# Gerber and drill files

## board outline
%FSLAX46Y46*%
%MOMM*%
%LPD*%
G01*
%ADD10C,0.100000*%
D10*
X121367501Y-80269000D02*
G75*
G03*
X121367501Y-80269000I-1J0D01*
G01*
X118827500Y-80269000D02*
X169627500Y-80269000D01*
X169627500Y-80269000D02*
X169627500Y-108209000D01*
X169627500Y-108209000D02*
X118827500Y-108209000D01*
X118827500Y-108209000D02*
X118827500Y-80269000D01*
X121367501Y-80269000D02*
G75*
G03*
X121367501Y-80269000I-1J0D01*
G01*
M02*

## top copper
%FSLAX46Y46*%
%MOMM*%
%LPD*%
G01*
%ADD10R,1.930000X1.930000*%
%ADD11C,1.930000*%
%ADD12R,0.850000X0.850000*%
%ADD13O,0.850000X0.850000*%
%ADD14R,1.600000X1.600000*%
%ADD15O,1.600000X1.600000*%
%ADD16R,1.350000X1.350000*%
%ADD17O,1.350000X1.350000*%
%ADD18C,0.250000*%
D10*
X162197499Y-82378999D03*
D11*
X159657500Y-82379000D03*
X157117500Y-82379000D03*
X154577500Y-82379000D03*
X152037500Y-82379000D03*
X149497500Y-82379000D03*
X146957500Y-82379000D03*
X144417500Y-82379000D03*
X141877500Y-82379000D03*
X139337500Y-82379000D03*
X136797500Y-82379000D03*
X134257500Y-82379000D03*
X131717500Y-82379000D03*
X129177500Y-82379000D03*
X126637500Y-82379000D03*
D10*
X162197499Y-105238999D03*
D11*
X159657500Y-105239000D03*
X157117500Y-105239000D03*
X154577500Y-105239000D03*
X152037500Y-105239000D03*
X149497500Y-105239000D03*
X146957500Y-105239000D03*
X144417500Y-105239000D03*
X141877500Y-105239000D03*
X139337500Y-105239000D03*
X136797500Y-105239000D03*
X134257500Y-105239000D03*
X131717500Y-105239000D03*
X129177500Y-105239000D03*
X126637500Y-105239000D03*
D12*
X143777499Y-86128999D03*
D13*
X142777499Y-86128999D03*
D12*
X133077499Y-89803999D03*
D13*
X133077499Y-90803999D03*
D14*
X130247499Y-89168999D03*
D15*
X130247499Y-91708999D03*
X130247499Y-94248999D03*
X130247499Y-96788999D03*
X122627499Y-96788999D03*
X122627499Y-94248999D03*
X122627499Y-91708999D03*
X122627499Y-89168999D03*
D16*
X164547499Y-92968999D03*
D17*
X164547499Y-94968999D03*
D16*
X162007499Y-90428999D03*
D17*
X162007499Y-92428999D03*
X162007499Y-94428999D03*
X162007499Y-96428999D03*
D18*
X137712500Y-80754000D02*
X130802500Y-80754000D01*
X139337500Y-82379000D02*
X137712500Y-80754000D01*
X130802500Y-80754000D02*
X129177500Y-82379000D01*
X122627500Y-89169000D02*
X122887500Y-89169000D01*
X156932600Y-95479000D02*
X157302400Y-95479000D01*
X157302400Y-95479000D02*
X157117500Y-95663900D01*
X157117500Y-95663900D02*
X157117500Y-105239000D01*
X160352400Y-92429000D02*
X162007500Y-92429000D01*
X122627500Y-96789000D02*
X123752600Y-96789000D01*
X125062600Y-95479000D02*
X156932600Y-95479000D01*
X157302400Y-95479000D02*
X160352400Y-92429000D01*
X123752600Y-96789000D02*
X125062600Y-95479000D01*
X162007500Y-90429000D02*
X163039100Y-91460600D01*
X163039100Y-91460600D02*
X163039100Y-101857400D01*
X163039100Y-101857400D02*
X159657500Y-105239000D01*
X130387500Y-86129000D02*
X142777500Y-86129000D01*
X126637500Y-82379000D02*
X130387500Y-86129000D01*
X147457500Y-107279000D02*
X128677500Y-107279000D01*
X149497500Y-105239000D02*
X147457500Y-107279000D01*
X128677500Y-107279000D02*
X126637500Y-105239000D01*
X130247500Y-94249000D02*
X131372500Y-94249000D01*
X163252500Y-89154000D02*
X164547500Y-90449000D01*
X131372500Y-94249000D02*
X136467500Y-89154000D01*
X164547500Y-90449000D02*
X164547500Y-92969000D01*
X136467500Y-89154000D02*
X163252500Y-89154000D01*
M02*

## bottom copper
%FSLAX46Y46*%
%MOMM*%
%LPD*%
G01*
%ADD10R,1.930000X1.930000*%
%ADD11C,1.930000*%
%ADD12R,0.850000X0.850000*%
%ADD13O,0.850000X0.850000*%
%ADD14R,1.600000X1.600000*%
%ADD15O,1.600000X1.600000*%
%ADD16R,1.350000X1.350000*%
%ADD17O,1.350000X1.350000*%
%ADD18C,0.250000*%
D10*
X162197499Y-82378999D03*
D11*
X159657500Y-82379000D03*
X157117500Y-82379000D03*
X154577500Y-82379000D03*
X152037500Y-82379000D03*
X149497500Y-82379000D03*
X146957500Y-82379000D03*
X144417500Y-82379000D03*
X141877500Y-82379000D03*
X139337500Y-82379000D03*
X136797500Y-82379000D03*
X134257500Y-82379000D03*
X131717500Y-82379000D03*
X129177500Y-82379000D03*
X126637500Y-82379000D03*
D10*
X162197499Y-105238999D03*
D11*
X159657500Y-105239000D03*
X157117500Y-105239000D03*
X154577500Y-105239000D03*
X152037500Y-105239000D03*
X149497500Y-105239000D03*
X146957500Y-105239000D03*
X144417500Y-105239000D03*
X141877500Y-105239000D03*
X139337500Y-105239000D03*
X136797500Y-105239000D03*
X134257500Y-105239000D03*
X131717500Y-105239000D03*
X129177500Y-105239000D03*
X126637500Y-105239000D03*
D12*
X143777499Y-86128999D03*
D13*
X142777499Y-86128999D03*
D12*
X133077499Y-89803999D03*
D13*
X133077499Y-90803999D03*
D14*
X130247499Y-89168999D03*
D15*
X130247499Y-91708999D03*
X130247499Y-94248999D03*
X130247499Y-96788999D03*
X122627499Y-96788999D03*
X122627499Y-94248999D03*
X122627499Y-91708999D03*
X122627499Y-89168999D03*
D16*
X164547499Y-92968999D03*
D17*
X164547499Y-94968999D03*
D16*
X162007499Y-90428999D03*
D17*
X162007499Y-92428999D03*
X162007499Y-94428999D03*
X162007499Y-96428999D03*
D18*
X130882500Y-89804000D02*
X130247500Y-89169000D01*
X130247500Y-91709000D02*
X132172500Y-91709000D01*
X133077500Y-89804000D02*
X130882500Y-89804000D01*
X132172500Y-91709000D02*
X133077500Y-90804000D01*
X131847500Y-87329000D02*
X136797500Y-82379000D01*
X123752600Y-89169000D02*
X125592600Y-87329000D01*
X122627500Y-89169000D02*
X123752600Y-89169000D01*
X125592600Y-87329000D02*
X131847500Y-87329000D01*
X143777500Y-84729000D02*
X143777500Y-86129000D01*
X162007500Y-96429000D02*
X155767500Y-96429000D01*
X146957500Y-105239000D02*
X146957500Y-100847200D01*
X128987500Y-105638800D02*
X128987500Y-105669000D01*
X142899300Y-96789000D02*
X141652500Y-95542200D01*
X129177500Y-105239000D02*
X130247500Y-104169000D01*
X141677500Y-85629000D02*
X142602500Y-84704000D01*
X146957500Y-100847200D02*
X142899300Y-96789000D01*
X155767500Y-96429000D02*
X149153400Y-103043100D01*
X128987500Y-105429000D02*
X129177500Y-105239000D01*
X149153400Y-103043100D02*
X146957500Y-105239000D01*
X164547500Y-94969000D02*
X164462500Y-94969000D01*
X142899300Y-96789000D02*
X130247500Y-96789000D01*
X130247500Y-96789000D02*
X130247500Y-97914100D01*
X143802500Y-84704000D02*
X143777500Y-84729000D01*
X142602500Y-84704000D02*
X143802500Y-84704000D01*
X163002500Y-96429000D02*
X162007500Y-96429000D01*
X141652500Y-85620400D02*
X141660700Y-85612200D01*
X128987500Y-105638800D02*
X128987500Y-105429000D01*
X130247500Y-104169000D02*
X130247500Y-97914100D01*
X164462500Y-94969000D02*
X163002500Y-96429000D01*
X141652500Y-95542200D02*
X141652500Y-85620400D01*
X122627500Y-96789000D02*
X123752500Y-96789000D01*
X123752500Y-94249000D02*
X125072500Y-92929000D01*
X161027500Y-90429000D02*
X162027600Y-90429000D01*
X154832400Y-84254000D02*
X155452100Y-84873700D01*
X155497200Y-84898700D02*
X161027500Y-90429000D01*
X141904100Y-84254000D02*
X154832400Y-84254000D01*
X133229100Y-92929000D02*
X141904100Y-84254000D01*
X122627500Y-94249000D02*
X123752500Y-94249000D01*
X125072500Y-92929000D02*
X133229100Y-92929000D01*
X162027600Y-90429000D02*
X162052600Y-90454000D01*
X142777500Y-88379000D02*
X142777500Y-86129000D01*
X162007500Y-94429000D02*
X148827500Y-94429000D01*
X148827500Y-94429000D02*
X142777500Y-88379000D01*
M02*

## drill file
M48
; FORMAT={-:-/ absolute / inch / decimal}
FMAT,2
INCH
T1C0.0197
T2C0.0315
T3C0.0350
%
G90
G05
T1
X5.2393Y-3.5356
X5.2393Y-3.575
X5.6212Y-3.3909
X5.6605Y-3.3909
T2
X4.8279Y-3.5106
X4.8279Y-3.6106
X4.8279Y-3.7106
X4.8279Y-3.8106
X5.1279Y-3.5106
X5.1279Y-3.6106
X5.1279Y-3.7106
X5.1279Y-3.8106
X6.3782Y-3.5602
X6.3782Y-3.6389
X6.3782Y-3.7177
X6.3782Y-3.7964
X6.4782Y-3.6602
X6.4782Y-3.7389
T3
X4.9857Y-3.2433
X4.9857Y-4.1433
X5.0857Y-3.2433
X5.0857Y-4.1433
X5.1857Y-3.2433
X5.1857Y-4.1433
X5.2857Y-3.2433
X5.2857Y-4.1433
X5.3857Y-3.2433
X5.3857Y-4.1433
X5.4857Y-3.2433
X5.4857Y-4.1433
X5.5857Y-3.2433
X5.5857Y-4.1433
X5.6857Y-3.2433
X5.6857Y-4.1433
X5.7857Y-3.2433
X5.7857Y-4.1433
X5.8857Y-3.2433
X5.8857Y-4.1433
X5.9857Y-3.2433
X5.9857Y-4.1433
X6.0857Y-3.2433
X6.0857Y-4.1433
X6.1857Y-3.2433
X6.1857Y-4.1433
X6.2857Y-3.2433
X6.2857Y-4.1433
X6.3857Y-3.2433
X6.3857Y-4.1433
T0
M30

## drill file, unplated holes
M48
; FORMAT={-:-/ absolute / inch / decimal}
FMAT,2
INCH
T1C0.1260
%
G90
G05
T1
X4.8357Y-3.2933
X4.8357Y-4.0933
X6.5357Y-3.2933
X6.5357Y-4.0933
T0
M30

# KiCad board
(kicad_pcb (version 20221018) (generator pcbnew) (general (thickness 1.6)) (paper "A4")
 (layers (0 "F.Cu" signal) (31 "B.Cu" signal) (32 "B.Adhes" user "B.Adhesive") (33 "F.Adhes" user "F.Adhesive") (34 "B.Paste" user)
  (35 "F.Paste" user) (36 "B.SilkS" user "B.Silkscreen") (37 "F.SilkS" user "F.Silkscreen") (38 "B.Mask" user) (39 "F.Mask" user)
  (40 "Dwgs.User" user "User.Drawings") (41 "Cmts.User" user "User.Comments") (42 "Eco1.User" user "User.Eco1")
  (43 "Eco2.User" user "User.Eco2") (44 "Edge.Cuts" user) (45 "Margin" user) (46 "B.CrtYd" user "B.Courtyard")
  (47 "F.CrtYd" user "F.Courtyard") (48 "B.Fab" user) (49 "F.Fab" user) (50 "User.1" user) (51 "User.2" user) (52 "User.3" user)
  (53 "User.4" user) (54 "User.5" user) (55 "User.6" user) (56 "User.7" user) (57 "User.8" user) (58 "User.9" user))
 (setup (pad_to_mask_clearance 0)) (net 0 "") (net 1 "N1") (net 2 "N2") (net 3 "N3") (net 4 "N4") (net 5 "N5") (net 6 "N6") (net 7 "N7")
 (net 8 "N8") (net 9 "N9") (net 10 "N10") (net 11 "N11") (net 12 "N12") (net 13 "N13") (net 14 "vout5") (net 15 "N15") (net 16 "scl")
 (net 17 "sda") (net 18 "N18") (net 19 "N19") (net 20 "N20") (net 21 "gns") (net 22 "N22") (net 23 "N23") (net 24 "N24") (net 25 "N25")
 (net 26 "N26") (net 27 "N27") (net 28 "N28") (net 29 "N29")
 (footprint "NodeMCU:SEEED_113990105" (layer "F.Cu") (at 144.4175 93.809 -90)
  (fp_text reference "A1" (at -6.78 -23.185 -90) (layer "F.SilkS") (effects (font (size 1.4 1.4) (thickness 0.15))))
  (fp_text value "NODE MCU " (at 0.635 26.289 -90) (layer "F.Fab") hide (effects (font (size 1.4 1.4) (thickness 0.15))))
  (pad "" np_thru_hole circle (at -10.16 -21.59 270) (size 3.2 3.2) (drill 3.2) (layers "*.Cu" "*.Mask"))
  (pad "" np_thru_hole circle (at -10.16 21.59 270) (size 3.2 3.2) (drill 3.2) (layers "*.Cu" "*.Mask"))
  (pad "" np_thru_hole circle (at 10.16 -21.59 270) (size 3.2 3.2) (drill 3.2) (layers "*.Cu" "*.Mask"))
  (pad "" np_thru_hole circle (at 10.16 21.59 270) (size 3.2 3.2) (drill 3.2) (layers "*.Cu" "*.Mask"))
  (pad "J1_1" thru_hole rect (at -11.43 -17.78 270) (size 1.93 1.93) (drill 0.889) (layers "*.Cu" "*.Mask") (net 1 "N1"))
  (pad "J1_2" thru_hole circle (at -11.43 -15.24 270) (size 1.93 1.93) (drill 0.889) (layers "*.Cu" "*.Mask") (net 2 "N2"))
  (pad "J1_3" thru_hole circle (at -11.43 -12.7 270) (size 1.93 1.93) (drill 0.889) (layers "*.Cu" "*.Mask") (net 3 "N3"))
  (pad "J1_4" thru_hole circle (at -11.43 -10.16 270) (size 1.93 1.93) (drill 0.889) (layers "*.Cu" "*.Mask") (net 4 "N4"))
  (pad "J1_5" thru_hole circle (at -11.43 -7.62 270) (size 1.93 1.93) (drill 0.889) (layers "*.Cu" "*.Mask") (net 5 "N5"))
  (pad "J1_6" thru_hole circle (at -11.43 -5.08 270) (size 1.93 1.93) (drill 0.889) (layers "*.Cu" "*.Mask") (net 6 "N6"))
  (pad "J1_7" thru_hole circle (at -11.43 -2.54 270) (size 1.93 1.93) (drill 0.889) (layers "*.Cu" "*.Mask") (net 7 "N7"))
  (pad "J1_8" thru_hole circle (at -11.43 0 270) (size 1.93 1.93) (drill 0.889) (layers "*.Cu" "*.Mask") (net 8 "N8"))
  (pad "J1_9" thru_hole circle (at -11.43 2.54 270) (size 1.93 1.93) (drill 0.889) (layers "*.Cu" "*.Mask") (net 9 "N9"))
  (pad "J1_10" thru_hole circle (at -11.43 5.08 270) (size 1.93 1.93) (drill 0.889) (layers "*.Cu" "*.Mask") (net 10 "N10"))
  (pad "J1_11" thru_hole circle (at -11.43 7.62 270) (size 1.93 1.93) (drill 0.889) (layers "*.Cu" "*.Mask") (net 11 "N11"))
  (pad "J1_12" thru_hole circle (at -11.43 10.16 270) (size 1.93 1.93) (drill 0.889) (layers "*.Cu" "*.Mask") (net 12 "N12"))
  (pad "J1_13" thru_hole circle (at -11.43 12.7 270) (size 1.93 1.93) (drill 0.889) (layers "*.Cu" "*.Mask") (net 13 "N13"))
  (pad "J1_14" thru_hole circle (at -11.43 15.24 270) (size 1.93 1.93) (drill 0.889) (layers "*.Cu" "*.Mask") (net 10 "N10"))
  (pad "J1_15" thru_hole circle (at -11.43 17.78 270) (size 1.93 1.93) (drill 0.889) (layers "*.Cu" "*.Mask") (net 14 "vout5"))
  (pad "J2_1" thru_hole rect (at 11.43 -17.78 270) (size 1.93 1.93) (drill 0.889) (layers "*.Cu" "*.Mask") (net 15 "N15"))
  (pad "J2_2" thru_hole circle (at 11.43 -15.24 270) (size 1.93 1.93) (drill 0.889) (layers "*.Cu" "*.Mask") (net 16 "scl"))
  (pad "J2_3" thru_hole circle (at 11.43 -12.7 270) (size 1.93 1.93) (drill 0.889) (layers "*.Cu" "*.Mask") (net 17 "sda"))
  (pad "J2_4" thru_hole circle (at 11.43 -10.16 270) (size 1.93 1.93) (drill 0.889) (layers "*.Cu" "*.Mask") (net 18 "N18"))
  (pad "J2_5" thru_hole circle (at 11.43 -7.62 270) (size 1.93 1.93) (drill 0.889) (layers "*.Cu" "*.Mask") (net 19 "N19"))
  (pad "J2_6" thru_hole circle (at 11.43 -5.08 270) (size 1.93 1.93) (drill 0.889) (layers "*.Cu" "*.Mask") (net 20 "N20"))
  (pad "J2_7" thru_hole circle (at 11.43 -2.54 270) (size 1.93 1.93) (drill 0.889) (layers "*.Cu" "*.Mask") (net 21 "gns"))
  (pad "J2_8" thru_hole circle (at 11.43 0 270) (size 1.93 1.93) (drill 0.889) (layers "*.Cu" "*.Mask") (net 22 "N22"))
  (pad "J2_9" thru_hole circle (at 11.43 2.54 270) (size 1.93 1.93) (drill 0.889) (layers "*.Cu" "*.Mask") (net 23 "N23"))
  (pad "J2_10" thru_hole circle (at 11.43 5.08 270) (size 1.93 1.93) (drill 0.889) (layers "*.Cu" "*.Mask") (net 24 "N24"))
  (pad "J2_11" thru_hole circle (at 11.43 7.62 270) (size 1.93 1.93) (drill 0.889) (layers "*.Cu" "*.Mask") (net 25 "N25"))
  (pad "J2_12" thru_hole circle (at 11.43 10.16 270) (size 1.93 1.93) (drill 0.889) (layers "*.Cu" "*.Mask") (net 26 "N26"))
  (pad "J2_13" thru_hole circle (at 11.43 12.7 270) (size 1.93 1.93) (drill 0.889) (layers "*.Cu" "*.Mask") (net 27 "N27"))
  (pad "J2_14" thru_hole circle (at 11.43 15.24 270) (size 1.93 1.93) (drill 0.889) (layers "*.Cu" "*.Mask") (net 21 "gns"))
  (pad "J2_15" thru_hole circle (at 11.43 17.78 270) (size 1.93 1.93) (drill 0.889) (layers "*.Cu" "*.Mask") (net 20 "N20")))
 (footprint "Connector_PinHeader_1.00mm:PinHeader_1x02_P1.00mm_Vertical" (layer "F.Cu") (at 143.7775 86.129 -90)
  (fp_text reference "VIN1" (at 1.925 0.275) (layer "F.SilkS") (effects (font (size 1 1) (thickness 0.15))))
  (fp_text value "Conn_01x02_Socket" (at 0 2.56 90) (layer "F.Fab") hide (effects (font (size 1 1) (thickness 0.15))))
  (pad "1" thru_hole rect (at 0 0 270) (size 0.85 0.85) (drill 0.5) (layers "*.Cu" "*.Mask") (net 21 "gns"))
  (pad "2" thru_hole oval (at 0 1 270) (size 0.85 0.85) (drill 0.5) (layers "*.Cu" "*.Mask") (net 14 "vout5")))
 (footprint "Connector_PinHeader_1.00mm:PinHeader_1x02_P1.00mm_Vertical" (layer "F.Cu") (at 133.0775 89.804)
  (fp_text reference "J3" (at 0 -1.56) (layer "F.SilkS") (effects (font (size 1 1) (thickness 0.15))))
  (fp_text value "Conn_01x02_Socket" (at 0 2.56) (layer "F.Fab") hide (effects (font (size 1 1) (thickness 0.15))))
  (pad "1" thru_hole rect (at 0 0) (size 0.85 0.85) (drill 0.5) (layers "*.Cu" "*.Mask"))
  (pad "2" thru_hole oval (at 0 1) (size 0.85 0.85) (drill 0.5) (layers "*.Cu" "*.Mask")))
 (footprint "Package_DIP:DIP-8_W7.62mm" (layer "B.Cu") (at 130.2475 89.169 180)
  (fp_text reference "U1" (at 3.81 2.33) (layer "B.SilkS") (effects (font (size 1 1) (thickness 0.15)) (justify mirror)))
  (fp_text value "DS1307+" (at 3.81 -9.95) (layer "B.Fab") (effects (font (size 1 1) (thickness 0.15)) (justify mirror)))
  (pad "1" thru_hole rect (at 0 0 180) (size 1.6 1.6) (drill 0.8) (layers "*.Cu" "*.Mask"))
  (pad "2" thru_hole oval (at 0 -2.54 180) (size 1.6 1.6) (drill 0.8) (layers "*.Cu" "*.Mask"))
  (pad "3" thru_hole oval (at 0 -5.08 180) (size 1.6 1.6) (drill 0.8) (layers "*.Cu" "*.Mask") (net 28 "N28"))
  (pad "4" thru_hole oval (at 0 -7.62 180) (size 1.6 1.6) (drill 0.8) (layers "*.Cu" "*.Mask") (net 21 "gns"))
  (pad "5" thru_hole oval (at 7.62 -7.62 180) (size 1.6 1.6) (drill 0.8) (layers "*.Cu" "*.Mask") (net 17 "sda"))
  (pad "6" thru_hole oval (at 7.62 -5.08 180) (size 1.6 1.6) (drill 0.8) (layers "*.Cu" "*.Mask") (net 16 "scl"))
  (pad "7" thru_hole oval (at 7.62 -2.54 180) (size 1.6 1.6) (drill 0.8) (layers "*.Cu" "*.Mask") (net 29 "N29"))
  (pad "8" thru_hole oval (at 7.62 0 180) (size 1.6 1.6) (drill 0.8) (layers "*.Cu" "*.Mask") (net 11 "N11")))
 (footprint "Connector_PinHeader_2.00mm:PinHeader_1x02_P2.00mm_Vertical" (layer "B.Cu") (at 164.5475 92.969 180)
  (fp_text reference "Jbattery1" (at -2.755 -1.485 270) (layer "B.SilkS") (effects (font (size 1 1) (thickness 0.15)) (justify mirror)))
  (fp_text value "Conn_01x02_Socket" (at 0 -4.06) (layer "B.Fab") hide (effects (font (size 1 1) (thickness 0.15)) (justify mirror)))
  (pad "1" thru_hole rect (at 0 0 180) (size 1.35 1.35) (drill 0.8) (layers "*.Cu" "*.Mask") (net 28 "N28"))
  (pad "2" thru_hole oval (at 0 -2 180) (size 1.35 1.35) (drill 0.8) (layers "*.Cu" "*.Mask") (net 21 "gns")))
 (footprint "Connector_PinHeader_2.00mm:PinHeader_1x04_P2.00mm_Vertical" (layer "B.Cu") (at 162.0075 90.429 180)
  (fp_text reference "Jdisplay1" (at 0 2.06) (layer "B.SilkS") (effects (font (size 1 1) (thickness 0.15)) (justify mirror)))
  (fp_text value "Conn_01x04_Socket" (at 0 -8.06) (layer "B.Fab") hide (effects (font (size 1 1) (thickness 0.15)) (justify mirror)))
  (pad "1" thru_hole rect (at 0 0 180) (size 1.35 1.35) (drill 0.8) (layers "*.Cu" "*.Mask") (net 16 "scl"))
  (pad "2" thru_hole oval (at 0 -2 180) (size 1.35 1.35) (drill 0.8) (layers "*.Cu" "*.Mask") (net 17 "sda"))
  (pad "3" thru_hole oval (at 0 -4 180) (size 1.35 1.35) (drill 0.8) (layers "*.Cu" "*.Mask") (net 14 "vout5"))
  (pad "4" thru_hole oval (at 0 -6 180) (size 1.35 1.35) (drill 0.8) (layers "*.Cu" "*.Mask") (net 21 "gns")))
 (gr_circle (center 121.3675 80.269) (end 121.3675 80.269) (stroke (width 0.1) (type default)) (fill none) (layer "Edge.Cuts"))
 (gr_rect (start 118.8275 80.269) (end 169.6275 108.209) (stroke (width 0.1) (type default)) (fill none) (layer "Edge.Cuts"))
 (gr_circle (center 121.3675 80.269) (end 121.3675 80.269) (stroke (width 0.1) (type default)) (fill none) (layer "Edge.Cuts"))
 (segment (start 130.8825 89.804) (end 130.2475 89.169) (width 0.25) (layer "B.Cu") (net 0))
 (segment (start 130.2475 91.709) (end 132.1725 91.709) (width 0.25) (layer "B.Cu") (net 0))
 (segment (start 133.0775 89.804) (end 130.8825 89.804) (width 0.25) (layer "B.Cu") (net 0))
 (segment (start 132.1725 91.709) (end 133.0775 90.804) (width 0.25) (layer "B.Cu") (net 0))
 (segment (start 137.7125 80.754) (end 130.8025 80.754) (width 0.25) (layer "F.Cu") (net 10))
 (segment (start 139.3375 82.379) (end 137.7125 80.754) (width 0.25) (layer "F.Cu") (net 10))
 (segment (start 130.8025 80.754) (end 129.1775 82.379) (width 0.25) (layer "F.Cu") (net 10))
 (segment (start 122.6275 89.169) (end 122.8875 89.169) (width 0.25) (layer "F.Cu") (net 11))
 (segment (start 131.8475 87.329) (end 136.7975 82.379) (width 0.25) (layer "B.Cu") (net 11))
 (segment (start 123.7526 89.169) (end 125.5926 87.329) (width 0.25) (layer "B.Cu") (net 11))
 (segment (start 122.6275 89.169) (end 123.7526 89.169) (width 0.25) (layer "B.Cu") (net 11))
 (segment (start 125.5926 87.329) (end 131.8475 87.329) (width 0.25) (layer "B.Cu") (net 11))
 (segment (start 143.7775 84.729) (end 143.7775 86.129) (width 0.25) (layer "B.Cu") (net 21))
 (segment (start 162.0075 96.429) (end 155.7675 96.429) (width 0.25) (layer "B.Cu") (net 21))
 (segment (start 146.9575 105.239) (end 146.9575 100.8472) (width 0.25) (layer "B.Cu") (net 21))
 (segment (start 128.9875 105.6388) (end 128.9875 105.669) (width 0.25) (layer "B.Cu") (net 21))
 (segment (start 142.8993 96.789) (end 141.6525 95.5422) (width 0.25) (layer "B.Cu") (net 21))
 (segment (start 129.1775 105.239) (end 130.2475 104.169) (width 0.25) (layer "B.Cu") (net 21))
 (segment (start 141.6775 85.629) (end 142.6025 84.704) (width 0.25) (layer "B.Cu") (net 21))
 (segment (start 146.9575 100.8472) (end 142.8993 96.789) (width 0.25) (layer "B.Cu") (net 21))
 (segment (start 155.7675 96.429) (end 149.1534 103.0431) (width 0.25) (layer "B.Cu") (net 21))
 (segment (start 128.9875 105.429) (end 129.1775 105.239) (width 0.25) (layer "B.Cu") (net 21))
 (segment (start 149.1534 103.0431) (end 146.9575 105.239) (width 0.25) (layer "B.Cu") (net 21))
 (segment (start 164.5475 94.969) (end 164.4625 94.969) (width 0.25) (layer "B.Cu") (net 21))
 (segment (start 142.8993 96.789) (end 130.2475 96.789) (width 0.25) (layer "B.Cu") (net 21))
 (segment (start 130.2475 96.789) (end 130.2475 97.9141) (width 0.25) (layer "B.Cu") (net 21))
 (segment (start 143.8025 84.704) (end 143.7775 84.729) (width 0.25) (layer "B.Cu") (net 21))
 (segment (start 142.6025 84.704) (end 143.8025 84.704) (width 0.25) (layer "B.Cu") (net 21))
 (segment (start 163.0025 96.429) (end 162.0075 96.429) (width 0.25) (layer "B.Cu") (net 21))
 (segment (start 141.6525 85.6204) (end 141.6607 85.6122) (width 0.25) (layer "B.Cu") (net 21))
 (segment (start 128.9875 105.6388) (end 128.9875 105.429) (width 0.25) (layer "B.Cu") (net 21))
 (segment (start 130.2475 104.169) (end 130.2475 97.9141) (width 0.25) (layer "B.Cu") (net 21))
 (segment (start 164.4625 94.969) (end 163.0025 96.429) (width 0.25) (layer "B.Cu") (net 21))
 (segment (start 141.6525 95.5422) (end 141.6525 85.6204) (width 0.25) (layer "B.Cu") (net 21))
 (segment (start 156.9326 95.479) (end 157.3024 95.479) (width 0.25) (layer "F.Cu") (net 17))
 (segment (start 157.3024 95.479) (end 157.1175 95.6639) (width 0.25) (layer "F.Cu") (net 17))
 (segment (start 157.1175 95.6639) (end 157.1175 105.239) (width 0.25) (layer "F.Cu") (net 17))
 (segment (start 160.3524 92.429) (end 162.0075 92.429) (width 0.25) (layer "F.Cu") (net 17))
 (segment (start 122.6275 96.789) (end 123.7526 96.789) (width 0.25) (layer "F.Cu") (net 17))
 (segment (start 125.0626 95.479) (end 156.9326 95.479) (width 0.25) (layer "F.Cu") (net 17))
 (segment (start 157.3024 95.479) (end 160.3524 92.429) (width 0.25) (layer "F.Cu") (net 17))
 (segment (start 123.7526 96.789) (end 125.0626 95.479) (width 0.25) (layer "F.Cu") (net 17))
 (segment (start 122.6275 96.789) (end 123.7525 96.789) (width 0.25) (layer "B.Cu") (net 17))
 (segment (start 162.0075 90.429) (end 163.0391 91.4606) (width 0.25) (layer "F.Cu") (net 16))
 (segment (start 163.0391 91.4606) (end 163.0391 101.8574) (width 0.25) (layer "F.Cu") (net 16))
 (segment (start 163.0391 101.8574) (end 159.6575 105.239) (width 0.25) (layer "F.Cu") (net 16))
 (segment (start 123.7525 94.249) (end 125.0725 92.929) (width 0.25) (layer "B.Cu") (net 16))
 (segment (start 161.0275 90.429) (end 162.0276 90.429) (width 0.25) (layer "B.Cu") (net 16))
 (segment (start 154.8324 84.254) (end 155.4521 84.8737) (width 0.25) (layer "B.Cu") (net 16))
 (segment (start 155.4972 84.8987) (end 161.0275 90.429) (width 0.25) (layer "B.Cu") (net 16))
 (segment (start 141.9041 84.254) (end 154.8324 84.254) (width 0.25) (layer "B.Cu") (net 16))
 (segment (start 133.2291 92.929) (end 141.9041 84.254) (width 0.25) (layer "B.Cu") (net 16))
 (segment (start 122.6275 94.249) (end 123.7525 94.249) (width 0.25) (layer "B.Cu") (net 16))
 (segment (start 125.0725 92.929) (end 133.2291 92.929) (width 0.25) (layer "B.Cu") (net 16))
 (segment (start 162.0276 90.429) (end 162.0526 90.454) (width 0.25) (layer "B.Cu") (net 16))
 (segment (start 130.3875 86.129) (end 142.7775 86.129) (width 0.25) (layer "F.Cu") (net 14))
 (segment (start 126.6375 82.379) (end 130.3875 86.129) (width 0.25) (layer "F.Cu") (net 14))
 (segment (start 142.7775 88.379) (end 142.7775 86.129) (width 0.25) (layer "B.Cu") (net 14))
 (segment (start 162.0075 94.429) (end 148.8275 94.429) (width 0.25) (layer "B.Cu") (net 14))
 (segment (start 148.8275 94.429) (end 142.7775 88.379) (width 0.25) (layer "B.Cu") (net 14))
 (segment (start 147.4575 107.279) (end 128.6775 107.279) (width 0.25) (layer "F.Cu") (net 20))
 (segment (start 149.4975 105.239) (end 147.4575 107.279) (width 0.25) (layer "F.Cu") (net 20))
 (segment (start 128.6775 107.279) (end 126.6375 105.239) (width 0.25) (layer "F.Cu") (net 20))
 (segment (start 130.2475 94.249) (end 131.3725 94.249) (width 0.25) (layer "F.Cu") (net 28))
 (segment (start 163.2525 89.154) (end 164.5475 90.449) (width 0.25) (layer "F.Cu") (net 28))
 (segment (start 131.3725 94.249) (end 136.4675 89.154) (width 0.25) (layer "F.Cu") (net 28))
 (segment (start 164.5475 90.449) (end 164.5475 92.969) (width 0.25) (layer "F.Cu") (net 28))
 (segment (start 136.4675 89.154) (end 163.2525 89.154) (width 0.25) (layer "F.Cu") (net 28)))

